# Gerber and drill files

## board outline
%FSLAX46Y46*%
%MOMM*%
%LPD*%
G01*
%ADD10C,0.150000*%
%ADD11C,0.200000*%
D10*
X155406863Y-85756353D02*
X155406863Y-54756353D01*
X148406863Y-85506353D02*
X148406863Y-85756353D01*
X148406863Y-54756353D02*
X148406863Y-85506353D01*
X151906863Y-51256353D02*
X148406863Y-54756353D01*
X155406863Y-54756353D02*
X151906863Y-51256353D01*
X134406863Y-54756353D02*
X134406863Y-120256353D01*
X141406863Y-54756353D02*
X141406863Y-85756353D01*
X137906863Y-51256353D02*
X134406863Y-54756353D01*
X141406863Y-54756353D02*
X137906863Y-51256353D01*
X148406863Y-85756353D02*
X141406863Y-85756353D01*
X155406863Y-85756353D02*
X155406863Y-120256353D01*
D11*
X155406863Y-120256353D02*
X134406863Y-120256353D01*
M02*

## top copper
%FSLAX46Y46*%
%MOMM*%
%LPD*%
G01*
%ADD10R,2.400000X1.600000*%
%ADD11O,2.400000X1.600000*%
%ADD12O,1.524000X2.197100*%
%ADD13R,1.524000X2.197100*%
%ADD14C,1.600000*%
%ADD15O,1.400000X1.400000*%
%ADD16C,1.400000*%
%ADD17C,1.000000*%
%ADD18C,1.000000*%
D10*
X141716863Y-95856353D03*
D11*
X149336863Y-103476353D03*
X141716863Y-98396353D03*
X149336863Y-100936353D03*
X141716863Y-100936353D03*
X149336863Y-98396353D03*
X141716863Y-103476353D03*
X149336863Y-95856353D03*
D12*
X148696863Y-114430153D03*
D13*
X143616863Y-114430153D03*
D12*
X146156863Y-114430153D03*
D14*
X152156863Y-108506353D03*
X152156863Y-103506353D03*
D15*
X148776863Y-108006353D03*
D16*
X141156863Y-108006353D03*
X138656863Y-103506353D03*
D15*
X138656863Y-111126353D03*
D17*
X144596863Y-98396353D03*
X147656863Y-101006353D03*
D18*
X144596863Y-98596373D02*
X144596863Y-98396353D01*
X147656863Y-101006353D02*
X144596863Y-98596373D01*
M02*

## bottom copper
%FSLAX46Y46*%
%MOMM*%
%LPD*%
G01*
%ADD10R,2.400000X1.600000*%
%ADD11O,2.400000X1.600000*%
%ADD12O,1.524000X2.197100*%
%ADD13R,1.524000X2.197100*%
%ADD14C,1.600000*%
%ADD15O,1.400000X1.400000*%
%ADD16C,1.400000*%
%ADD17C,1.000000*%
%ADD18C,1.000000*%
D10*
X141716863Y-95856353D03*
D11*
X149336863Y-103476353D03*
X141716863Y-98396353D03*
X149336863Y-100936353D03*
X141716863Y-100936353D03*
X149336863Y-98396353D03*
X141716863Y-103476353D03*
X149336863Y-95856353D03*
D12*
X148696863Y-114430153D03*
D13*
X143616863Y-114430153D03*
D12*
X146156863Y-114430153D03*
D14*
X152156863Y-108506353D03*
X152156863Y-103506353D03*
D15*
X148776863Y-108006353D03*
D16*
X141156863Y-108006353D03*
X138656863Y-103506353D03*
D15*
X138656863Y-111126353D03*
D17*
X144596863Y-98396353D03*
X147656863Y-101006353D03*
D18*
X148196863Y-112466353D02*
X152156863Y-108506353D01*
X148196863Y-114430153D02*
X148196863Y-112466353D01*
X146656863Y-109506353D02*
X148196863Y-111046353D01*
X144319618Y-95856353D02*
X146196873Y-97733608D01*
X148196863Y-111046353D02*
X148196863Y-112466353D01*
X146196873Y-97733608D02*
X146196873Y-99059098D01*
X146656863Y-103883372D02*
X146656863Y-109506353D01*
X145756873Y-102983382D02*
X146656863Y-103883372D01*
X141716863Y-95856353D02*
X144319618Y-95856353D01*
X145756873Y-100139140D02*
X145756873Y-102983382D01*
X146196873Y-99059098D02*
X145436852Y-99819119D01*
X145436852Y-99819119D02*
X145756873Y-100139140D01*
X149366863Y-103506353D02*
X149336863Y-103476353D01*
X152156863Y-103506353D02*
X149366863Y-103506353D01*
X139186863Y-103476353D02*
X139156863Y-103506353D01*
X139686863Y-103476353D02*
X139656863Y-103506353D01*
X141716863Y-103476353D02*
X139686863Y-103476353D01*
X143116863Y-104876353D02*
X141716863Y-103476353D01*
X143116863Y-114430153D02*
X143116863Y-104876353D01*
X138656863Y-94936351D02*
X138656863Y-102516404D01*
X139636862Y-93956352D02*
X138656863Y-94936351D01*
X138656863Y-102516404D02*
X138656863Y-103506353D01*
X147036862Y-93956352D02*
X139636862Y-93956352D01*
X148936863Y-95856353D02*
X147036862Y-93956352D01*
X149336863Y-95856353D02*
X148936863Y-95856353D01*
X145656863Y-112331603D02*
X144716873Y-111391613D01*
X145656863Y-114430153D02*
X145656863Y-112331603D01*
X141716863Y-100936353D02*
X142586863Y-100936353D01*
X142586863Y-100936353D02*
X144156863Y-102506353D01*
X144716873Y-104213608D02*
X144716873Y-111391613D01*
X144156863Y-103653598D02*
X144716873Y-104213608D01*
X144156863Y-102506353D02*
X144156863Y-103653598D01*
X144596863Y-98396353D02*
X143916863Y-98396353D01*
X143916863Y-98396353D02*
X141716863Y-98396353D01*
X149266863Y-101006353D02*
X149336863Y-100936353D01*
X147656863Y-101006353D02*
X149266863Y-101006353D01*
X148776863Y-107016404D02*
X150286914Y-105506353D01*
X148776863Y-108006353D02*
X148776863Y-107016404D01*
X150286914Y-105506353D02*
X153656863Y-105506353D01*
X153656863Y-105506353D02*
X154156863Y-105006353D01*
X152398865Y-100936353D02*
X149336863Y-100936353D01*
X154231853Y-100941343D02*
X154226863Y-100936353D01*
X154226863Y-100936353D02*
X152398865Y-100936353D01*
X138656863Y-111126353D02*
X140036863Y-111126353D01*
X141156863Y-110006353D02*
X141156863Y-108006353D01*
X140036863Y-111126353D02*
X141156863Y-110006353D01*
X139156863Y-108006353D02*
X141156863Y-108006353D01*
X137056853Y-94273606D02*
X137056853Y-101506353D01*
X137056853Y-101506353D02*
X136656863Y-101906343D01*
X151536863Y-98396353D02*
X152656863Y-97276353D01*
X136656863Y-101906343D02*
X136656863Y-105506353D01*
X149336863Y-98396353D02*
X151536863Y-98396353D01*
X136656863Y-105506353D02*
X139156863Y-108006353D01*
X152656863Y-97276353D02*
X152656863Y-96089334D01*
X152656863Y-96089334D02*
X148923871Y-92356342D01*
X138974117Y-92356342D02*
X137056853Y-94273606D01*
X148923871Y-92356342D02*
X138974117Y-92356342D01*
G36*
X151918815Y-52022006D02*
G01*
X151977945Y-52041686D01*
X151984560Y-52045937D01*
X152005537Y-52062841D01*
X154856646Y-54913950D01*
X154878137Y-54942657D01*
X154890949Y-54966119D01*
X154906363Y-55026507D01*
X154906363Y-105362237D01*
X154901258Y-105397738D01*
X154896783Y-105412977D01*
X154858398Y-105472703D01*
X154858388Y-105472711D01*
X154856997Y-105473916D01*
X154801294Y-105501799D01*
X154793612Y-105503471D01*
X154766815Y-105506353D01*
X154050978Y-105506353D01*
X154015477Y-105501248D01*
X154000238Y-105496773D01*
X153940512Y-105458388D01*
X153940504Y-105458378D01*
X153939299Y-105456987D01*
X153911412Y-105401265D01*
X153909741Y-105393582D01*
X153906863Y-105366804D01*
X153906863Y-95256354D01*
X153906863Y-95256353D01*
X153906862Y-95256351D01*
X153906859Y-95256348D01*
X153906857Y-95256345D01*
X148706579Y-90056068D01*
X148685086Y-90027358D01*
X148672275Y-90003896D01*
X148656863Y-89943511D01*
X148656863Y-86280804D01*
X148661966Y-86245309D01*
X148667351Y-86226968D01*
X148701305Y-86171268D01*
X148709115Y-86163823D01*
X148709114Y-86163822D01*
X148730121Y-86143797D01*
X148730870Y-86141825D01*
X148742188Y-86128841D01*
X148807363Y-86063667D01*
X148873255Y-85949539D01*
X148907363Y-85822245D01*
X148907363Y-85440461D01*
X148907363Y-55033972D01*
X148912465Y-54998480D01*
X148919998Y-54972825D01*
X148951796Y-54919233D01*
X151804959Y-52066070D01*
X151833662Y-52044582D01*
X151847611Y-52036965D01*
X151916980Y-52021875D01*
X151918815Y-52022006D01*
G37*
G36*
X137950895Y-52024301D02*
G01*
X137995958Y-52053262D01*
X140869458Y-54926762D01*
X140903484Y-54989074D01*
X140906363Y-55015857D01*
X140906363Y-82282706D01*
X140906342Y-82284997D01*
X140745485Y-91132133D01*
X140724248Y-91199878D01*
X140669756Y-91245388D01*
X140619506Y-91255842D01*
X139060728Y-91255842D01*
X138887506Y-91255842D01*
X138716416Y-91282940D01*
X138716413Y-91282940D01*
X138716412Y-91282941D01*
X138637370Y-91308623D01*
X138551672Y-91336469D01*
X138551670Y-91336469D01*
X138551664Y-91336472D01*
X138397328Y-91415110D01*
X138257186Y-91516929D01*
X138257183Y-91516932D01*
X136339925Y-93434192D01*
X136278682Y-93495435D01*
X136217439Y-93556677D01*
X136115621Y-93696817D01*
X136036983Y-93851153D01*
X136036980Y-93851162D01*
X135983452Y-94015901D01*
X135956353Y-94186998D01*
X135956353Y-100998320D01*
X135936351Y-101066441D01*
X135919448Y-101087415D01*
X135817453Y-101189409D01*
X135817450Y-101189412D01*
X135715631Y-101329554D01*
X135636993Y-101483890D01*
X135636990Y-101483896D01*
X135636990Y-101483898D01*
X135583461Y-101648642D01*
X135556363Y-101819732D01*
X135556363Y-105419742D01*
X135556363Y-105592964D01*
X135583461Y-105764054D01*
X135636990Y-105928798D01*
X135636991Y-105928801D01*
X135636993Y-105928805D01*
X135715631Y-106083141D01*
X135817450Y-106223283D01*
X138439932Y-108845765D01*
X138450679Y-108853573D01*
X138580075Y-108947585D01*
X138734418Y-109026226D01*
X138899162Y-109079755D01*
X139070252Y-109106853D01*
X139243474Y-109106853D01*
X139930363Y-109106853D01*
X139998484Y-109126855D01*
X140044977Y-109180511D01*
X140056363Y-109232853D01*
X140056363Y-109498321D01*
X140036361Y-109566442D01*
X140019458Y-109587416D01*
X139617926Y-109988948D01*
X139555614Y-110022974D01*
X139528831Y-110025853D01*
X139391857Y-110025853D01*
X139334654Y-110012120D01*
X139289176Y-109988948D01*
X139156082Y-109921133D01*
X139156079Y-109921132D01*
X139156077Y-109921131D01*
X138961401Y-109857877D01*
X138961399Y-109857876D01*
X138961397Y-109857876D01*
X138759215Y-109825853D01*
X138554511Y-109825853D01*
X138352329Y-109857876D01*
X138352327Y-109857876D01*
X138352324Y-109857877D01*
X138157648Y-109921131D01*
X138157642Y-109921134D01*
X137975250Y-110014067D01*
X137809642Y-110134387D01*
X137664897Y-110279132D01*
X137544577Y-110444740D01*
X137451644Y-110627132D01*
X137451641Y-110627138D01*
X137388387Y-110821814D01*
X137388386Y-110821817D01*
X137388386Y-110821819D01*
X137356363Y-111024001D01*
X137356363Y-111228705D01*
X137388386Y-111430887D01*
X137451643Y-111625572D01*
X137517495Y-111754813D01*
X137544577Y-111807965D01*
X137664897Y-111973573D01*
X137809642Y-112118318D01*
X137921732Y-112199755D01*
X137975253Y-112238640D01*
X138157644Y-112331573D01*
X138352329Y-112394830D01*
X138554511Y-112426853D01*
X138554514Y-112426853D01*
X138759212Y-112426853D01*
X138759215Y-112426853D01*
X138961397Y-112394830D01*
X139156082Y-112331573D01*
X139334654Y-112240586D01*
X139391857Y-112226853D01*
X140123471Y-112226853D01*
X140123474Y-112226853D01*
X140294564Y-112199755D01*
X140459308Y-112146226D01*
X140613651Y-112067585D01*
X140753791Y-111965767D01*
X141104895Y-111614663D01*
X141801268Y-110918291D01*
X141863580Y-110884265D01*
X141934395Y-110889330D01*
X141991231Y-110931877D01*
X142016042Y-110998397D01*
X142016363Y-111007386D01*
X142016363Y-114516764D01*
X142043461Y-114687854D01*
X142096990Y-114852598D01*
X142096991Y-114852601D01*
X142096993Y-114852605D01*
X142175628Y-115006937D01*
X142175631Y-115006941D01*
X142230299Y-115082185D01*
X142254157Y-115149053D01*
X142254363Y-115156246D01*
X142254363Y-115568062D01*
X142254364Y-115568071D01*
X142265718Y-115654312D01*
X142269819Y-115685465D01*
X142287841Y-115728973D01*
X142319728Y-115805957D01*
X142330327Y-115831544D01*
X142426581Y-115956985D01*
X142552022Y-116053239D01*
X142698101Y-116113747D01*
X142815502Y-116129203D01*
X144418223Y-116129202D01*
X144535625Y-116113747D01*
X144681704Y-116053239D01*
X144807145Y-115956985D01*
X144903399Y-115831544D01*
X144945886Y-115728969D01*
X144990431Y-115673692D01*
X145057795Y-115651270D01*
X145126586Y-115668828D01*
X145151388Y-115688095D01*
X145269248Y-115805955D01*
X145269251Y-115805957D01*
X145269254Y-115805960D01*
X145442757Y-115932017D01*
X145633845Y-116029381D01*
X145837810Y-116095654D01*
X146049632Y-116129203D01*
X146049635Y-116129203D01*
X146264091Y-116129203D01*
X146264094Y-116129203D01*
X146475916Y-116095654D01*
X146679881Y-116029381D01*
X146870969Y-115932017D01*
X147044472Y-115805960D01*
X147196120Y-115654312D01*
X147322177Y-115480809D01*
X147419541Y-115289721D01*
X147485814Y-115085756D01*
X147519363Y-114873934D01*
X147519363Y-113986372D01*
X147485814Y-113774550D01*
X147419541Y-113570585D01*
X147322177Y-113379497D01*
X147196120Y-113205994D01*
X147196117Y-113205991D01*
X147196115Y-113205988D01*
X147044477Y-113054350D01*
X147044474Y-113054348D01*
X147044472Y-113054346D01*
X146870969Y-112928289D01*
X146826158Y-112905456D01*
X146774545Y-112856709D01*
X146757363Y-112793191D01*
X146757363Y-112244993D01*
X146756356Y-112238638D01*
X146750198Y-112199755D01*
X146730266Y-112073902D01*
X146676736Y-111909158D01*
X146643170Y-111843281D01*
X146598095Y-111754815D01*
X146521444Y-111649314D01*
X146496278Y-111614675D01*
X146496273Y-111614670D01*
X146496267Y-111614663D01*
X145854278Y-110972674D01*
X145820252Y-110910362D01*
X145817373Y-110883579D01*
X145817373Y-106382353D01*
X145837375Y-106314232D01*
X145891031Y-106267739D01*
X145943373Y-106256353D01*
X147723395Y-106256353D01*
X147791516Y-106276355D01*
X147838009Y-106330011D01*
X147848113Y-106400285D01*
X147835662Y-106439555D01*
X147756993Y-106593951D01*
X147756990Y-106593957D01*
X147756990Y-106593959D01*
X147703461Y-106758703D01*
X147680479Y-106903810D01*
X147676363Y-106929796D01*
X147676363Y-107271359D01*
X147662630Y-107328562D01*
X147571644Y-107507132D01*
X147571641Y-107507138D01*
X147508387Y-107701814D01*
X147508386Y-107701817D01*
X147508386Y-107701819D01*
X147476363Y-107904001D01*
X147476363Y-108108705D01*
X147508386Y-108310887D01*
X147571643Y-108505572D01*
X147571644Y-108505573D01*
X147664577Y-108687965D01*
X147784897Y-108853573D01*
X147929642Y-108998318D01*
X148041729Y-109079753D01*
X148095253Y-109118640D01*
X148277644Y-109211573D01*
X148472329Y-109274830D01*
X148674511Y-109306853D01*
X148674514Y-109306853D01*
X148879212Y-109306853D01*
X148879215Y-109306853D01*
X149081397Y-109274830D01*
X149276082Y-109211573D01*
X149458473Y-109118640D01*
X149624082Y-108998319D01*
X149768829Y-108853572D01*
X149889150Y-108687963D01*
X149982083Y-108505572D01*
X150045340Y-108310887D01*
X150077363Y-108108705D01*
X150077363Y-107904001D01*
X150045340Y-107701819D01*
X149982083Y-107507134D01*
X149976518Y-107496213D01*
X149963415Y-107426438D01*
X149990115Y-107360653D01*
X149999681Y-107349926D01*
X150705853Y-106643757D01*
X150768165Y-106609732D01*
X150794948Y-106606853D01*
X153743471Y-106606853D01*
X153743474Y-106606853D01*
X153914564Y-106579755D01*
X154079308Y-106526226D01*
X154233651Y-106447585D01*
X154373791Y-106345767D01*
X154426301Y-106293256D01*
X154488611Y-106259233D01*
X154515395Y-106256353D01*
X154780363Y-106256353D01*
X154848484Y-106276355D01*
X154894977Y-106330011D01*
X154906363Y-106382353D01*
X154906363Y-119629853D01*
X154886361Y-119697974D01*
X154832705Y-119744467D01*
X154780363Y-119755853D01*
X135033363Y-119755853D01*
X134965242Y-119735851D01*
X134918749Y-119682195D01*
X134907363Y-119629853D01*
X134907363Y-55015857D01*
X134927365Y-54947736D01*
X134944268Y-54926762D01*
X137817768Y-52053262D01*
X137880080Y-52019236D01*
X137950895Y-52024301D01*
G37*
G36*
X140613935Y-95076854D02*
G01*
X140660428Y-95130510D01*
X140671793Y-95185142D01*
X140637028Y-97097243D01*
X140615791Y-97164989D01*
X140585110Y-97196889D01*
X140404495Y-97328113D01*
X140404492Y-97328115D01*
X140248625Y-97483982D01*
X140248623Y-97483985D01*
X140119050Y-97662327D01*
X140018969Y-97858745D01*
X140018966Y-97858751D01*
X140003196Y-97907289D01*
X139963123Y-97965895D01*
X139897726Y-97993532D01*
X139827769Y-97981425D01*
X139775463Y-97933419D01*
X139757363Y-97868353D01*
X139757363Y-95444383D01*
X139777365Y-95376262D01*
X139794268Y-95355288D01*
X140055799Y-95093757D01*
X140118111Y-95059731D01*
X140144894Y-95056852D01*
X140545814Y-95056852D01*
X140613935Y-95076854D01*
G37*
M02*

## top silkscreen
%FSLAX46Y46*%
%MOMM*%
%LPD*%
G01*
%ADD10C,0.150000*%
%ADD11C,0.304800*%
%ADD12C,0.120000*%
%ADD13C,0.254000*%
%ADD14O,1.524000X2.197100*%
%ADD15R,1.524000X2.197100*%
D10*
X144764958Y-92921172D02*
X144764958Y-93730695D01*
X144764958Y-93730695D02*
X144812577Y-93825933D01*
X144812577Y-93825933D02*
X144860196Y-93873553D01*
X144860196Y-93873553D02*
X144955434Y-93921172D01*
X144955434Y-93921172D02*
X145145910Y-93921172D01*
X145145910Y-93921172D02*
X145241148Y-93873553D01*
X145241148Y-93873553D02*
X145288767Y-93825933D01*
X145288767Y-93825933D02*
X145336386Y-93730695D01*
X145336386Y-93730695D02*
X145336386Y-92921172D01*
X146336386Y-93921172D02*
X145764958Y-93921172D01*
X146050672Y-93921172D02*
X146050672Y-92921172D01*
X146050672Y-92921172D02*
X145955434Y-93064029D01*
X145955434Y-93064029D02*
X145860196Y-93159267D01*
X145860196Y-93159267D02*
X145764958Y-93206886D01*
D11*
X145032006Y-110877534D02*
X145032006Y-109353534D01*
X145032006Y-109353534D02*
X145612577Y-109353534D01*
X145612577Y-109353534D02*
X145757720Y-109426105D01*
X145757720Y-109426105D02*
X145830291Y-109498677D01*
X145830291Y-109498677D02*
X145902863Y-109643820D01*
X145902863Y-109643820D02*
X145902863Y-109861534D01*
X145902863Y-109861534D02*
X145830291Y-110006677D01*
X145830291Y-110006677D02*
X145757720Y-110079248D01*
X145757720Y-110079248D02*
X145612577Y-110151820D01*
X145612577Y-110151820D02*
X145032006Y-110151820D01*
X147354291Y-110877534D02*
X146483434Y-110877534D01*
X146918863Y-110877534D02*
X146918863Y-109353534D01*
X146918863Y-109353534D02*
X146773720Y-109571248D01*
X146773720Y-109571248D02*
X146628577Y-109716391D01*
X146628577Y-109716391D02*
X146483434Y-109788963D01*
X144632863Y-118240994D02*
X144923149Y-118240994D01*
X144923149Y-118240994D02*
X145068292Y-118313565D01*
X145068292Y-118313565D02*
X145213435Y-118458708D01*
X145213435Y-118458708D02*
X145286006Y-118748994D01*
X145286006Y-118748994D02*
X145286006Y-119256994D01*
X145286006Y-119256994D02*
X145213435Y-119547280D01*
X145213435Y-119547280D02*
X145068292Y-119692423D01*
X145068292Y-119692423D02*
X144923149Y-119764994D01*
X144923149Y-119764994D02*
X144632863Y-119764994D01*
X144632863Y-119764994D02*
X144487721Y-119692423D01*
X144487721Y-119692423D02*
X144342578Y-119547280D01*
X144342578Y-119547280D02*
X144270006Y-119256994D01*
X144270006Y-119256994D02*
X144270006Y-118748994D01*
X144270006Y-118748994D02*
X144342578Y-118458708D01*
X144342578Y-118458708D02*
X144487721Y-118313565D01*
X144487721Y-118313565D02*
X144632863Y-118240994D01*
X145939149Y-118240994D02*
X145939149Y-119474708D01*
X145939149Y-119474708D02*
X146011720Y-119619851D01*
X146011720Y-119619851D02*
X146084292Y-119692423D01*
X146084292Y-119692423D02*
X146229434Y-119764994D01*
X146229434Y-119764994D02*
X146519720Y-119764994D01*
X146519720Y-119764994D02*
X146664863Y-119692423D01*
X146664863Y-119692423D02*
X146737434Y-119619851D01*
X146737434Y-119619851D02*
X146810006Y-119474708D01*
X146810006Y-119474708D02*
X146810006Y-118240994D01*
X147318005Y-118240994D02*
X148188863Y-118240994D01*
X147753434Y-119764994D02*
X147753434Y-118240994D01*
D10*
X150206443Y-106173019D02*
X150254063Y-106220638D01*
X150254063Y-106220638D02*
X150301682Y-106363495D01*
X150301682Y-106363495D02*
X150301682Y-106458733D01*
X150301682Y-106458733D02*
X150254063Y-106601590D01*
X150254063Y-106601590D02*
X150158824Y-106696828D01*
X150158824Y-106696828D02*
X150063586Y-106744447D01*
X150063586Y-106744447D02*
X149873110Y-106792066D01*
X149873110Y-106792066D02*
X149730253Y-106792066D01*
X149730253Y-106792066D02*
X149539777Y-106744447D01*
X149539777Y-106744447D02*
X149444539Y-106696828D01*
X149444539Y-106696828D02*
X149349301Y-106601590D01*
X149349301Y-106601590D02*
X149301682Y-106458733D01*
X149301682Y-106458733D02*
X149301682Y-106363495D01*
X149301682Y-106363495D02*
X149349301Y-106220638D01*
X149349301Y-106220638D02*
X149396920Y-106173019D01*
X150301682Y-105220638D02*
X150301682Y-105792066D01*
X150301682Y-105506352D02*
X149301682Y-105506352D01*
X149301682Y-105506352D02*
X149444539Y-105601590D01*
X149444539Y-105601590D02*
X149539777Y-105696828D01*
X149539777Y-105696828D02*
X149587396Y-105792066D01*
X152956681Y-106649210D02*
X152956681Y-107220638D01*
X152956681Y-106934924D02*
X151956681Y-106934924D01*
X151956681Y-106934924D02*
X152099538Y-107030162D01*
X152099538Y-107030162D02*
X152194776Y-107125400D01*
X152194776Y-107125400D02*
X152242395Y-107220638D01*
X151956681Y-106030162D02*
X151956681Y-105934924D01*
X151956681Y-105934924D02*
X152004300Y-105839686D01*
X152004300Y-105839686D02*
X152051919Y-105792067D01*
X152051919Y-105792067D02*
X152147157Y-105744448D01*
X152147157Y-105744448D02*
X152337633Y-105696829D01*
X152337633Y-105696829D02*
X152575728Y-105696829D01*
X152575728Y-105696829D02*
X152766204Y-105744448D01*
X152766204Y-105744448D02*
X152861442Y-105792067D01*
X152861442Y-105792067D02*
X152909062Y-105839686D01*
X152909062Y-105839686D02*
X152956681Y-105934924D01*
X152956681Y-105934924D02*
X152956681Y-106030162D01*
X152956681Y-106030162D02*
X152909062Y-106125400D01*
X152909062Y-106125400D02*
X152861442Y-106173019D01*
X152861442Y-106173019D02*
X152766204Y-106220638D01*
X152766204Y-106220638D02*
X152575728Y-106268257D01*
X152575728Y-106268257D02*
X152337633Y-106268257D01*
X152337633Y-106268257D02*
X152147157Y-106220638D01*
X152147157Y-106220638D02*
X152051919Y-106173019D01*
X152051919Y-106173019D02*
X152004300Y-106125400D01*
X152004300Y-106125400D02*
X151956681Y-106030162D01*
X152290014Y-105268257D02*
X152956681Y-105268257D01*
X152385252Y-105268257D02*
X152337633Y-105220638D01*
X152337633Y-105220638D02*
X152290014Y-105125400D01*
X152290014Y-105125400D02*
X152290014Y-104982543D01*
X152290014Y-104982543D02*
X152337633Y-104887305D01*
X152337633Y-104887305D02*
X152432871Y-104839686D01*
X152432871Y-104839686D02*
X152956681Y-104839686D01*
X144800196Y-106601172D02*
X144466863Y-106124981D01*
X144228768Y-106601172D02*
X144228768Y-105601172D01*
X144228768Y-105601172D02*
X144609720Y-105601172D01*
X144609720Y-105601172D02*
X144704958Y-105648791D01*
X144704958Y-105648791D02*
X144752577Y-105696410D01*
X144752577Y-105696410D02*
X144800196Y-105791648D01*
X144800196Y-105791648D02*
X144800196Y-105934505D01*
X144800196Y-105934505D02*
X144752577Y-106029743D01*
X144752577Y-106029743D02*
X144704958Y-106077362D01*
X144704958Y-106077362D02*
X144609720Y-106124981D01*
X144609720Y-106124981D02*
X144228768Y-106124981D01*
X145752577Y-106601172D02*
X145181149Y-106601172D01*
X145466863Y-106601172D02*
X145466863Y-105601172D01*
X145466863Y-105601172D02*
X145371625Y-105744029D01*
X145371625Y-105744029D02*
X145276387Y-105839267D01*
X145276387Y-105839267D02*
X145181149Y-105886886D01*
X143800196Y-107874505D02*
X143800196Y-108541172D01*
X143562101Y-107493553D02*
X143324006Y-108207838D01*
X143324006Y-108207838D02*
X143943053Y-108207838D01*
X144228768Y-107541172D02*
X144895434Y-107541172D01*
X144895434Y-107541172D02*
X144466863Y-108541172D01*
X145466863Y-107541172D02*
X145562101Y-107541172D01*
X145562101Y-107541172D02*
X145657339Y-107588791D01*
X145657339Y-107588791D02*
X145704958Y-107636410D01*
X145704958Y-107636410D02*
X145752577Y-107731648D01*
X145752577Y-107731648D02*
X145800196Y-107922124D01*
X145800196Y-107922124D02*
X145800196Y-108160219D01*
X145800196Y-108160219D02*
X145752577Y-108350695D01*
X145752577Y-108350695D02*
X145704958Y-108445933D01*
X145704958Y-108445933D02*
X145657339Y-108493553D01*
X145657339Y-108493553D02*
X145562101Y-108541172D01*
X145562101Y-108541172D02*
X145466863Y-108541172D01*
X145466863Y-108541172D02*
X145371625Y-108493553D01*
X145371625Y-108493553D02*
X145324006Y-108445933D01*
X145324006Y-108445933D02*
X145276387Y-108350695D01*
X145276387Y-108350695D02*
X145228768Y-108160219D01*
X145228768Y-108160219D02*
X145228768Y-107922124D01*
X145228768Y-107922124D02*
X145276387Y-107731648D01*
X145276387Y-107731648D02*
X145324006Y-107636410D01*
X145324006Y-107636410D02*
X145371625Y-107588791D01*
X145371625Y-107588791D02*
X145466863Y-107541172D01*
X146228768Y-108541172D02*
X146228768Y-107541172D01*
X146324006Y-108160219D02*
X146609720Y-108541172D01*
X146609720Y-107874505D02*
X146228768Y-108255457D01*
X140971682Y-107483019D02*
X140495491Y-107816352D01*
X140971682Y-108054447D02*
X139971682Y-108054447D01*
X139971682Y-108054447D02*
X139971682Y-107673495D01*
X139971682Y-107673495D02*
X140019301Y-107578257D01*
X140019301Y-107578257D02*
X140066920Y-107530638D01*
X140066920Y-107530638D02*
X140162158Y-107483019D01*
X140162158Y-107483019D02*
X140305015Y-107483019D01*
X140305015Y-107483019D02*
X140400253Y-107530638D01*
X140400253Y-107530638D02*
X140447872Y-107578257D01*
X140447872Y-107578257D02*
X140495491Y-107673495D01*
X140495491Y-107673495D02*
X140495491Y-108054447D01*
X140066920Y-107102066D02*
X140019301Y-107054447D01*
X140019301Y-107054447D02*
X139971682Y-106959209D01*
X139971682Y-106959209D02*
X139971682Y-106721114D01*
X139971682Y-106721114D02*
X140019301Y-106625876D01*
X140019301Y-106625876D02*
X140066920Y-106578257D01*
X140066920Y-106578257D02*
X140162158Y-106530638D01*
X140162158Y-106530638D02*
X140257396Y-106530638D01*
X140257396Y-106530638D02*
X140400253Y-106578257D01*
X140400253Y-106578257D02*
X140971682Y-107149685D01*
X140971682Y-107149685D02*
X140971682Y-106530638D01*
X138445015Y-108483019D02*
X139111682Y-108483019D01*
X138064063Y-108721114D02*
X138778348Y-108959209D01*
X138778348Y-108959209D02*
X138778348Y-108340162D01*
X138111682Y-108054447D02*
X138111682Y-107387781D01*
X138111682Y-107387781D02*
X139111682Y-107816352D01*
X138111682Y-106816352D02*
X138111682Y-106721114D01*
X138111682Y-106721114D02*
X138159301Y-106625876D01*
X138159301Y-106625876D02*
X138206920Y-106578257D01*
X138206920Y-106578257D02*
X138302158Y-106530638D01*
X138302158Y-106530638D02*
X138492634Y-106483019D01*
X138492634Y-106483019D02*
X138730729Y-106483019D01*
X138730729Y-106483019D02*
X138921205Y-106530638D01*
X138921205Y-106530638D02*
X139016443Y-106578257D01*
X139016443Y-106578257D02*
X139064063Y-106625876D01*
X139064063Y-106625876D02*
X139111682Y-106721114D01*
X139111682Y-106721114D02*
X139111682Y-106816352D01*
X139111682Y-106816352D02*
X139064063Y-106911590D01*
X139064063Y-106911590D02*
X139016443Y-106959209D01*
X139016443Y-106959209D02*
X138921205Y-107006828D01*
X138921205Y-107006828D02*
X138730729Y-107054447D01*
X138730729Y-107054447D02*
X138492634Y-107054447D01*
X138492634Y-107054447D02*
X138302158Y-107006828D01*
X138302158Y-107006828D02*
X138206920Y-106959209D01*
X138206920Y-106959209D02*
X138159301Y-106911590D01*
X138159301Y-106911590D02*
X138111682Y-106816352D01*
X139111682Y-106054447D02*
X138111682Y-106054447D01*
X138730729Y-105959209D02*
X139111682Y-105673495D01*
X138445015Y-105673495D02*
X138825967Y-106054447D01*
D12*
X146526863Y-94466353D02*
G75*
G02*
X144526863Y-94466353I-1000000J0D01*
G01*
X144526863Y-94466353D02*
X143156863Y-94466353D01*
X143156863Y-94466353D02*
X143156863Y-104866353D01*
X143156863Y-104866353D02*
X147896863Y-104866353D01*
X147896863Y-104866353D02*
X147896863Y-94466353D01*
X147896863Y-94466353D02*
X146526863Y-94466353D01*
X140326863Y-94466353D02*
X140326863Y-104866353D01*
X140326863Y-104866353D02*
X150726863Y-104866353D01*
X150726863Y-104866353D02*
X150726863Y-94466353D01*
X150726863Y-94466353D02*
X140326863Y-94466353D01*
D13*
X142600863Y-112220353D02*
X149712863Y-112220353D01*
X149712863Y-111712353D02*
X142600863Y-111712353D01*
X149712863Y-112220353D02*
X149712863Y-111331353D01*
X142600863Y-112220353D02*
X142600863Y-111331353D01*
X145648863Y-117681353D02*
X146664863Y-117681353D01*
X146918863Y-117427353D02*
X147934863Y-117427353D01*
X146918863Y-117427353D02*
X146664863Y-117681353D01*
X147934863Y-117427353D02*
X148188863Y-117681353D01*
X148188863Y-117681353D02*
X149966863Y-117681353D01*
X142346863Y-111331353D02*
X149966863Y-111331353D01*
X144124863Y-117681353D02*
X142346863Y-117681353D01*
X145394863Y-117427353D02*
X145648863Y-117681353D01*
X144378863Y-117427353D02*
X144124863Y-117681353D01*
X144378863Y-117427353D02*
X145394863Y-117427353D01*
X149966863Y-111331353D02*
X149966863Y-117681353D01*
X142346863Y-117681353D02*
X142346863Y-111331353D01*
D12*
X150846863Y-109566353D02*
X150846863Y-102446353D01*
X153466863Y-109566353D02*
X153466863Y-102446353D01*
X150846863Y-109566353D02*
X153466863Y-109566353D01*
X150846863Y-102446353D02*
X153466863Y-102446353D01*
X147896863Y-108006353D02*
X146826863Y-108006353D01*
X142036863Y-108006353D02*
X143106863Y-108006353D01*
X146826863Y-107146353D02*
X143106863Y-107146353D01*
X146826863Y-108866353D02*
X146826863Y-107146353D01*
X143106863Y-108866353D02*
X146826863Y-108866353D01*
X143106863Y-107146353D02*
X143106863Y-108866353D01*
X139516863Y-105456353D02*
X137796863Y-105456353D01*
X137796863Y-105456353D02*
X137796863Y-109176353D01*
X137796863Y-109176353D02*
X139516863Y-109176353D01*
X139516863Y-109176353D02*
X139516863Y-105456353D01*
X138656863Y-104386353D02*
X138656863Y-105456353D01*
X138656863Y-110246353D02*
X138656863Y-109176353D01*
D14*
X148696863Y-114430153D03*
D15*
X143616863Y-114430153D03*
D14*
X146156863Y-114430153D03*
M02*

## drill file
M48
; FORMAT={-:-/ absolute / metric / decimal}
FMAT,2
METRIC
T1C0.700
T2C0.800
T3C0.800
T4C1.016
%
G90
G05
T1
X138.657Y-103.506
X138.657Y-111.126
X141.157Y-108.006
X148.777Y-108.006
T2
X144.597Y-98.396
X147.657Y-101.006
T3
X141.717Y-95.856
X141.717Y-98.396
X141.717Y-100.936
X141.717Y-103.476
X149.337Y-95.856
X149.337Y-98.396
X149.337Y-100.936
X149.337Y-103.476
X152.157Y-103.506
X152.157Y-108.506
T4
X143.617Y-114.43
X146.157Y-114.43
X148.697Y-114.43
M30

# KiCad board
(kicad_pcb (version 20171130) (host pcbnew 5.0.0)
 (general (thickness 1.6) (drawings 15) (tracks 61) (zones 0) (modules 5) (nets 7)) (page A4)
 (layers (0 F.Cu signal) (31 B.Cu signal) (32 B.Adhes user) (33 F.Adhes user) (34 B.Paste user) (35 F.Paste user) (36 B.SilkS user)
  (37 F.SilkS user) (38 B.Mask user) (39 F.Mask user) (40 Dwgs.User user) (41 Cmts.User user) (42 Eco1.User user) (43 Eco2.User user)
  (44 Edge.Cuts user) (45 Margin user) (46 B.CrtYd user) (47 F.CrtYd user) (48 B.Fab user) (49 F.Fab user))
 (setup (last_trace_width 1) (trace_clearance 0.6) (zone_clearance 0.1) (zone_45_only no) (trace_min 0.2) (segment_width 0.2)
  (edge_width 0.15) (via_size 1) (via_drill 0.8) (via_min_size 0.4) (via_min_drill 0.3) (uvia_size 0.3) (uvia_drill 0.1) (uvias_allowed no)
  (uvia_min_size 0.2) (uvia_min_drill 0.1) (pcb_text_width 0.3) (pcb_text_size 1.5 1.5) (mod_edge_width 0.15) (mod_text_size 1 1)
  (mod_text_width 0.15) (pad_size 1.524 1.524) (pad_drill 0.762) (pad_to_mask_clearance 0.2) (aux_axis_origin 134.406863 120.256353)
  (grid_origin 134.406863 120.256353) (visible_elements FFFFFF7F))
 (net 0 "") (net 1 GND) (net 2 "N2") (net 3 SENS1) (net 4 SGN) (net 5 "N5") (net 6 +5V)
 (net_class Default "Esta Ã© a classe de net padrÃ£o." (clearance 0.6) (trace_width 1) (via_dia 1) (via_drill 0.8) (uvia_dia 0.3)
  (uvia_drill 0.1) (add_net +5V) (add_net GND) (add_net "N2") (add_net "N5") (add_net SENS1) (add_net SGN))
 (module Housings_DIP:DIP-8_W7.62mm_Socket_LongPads (layer F.Cu) (at 141.716863 95.856353)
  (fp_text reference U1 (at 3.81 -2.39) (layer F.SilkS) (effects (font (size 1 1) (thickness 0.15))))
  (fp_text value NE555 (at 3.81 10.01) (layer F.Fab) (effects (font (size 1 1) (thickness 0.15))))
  (fp_arc (start 3.81 -1.39) (end 2.81 -1.39) (angle -180) (layer F.SilkS) (width 0.12))
  (fp_line (start 2.81 -1.39) (end 1.44 -1.39) (layer F.SilkS) (width 0.12))
  (fp_line (start 1.44 -1.39) (end 1.44 9.01) (layer F.SilkS) (width 0.12))
  (fp_line (start 1.44 9.01) (end 6.18 9.01) (layer F.SilkS) (width 0.12))
  (fp_line (start 6.18 9.01) (end 6.18 -1.39) (layer F.SilkS) (width 0.12))
  (fp_line (start 6.18 -1.39) (end 4.81 -1.39) (layer F.SilkS) (width 0.12))
  (fp_line (start -1.39 -1.39) (end -1.39 9.01) (layer F.SilkS) (width 0.12))
  (fp_line (start -1.39 9.01) (end 9.01 9.01) (layer F.SilkS) (width 0.12))
  (fp_line (start 9.01 9.01) (end 9.01 -1.39) (layer F.SilkS) (width 0.12))
  (fp_line (start 9.01 -1.39) (end -1.39 -1.39) (layer F.SilkS) (width 0.12))
  (pad 1 thru_hole rect (at 0 0) (size 2.4 1.6) (drill 0.8) (layers *.Mask B.Cu) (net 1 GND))
  (pad 5 thru_hole oval (at 7.62 7.62) (size 2.4 1.6) (drill 0.8) (layers *.Mask B.Cu) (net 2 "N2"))
  (pad 2 thru_hole oval (at 0 2.54) (size 2.4 1.6) (drill 0.8) (layers *.Mask B.Cu) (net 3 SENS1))
  (pad 6 thru_hole oval (at 7.62 5.08) (size 2.4 1.6) (drill 0.8) (layers *.Mask B.Cu) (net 3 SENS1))
  (pad 3 thru_hole oval (at 0 5.08) (size 2.4 1.6) (drill 0.8) (layers *.Mask B.Cu) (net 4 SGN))
  (pad 7 thru_hole oval (at 7.62 2.54) (size 2.4 1.6) (drill 0.8) (layers *.Mask B.Cu) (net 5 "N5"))
  (pad 4 thru_hole oval (at 0 7.62) (size 2.4 1.6) (drill 0.8) (layers *.Mask B.Cu) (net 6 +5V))
  (pad 8 thru_hole oval (at 7.62 0) (size 2.4 1.6) (drill 0.8) (layers *.Mask B.Cu) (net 6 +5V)))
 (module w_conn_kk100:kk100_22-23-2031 (layer F.Cu) (at 146.156863 114.506353)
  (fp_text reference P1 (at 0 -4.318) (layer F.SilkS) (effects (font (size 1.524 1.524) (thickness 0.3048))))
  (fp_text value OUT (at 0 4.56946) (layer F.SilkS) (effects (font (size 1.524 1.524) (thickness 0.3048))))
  (fp_line (start -3.556 -2.286) (end 3.556 -2.286) (layer F.SilkS) (width 0.254))
  (fp_line (start 3.556 -2.794) (end -3.556 -2.794) (layer F.SilkS) (width 0.254))
  (fp_line (start 3.556 -2.286) (end 3.556 -3.175) (layer F.SilkS) (width 0.254))
  (fp_line (start -3.556 -2.286) (end -3.556 -3.175) (layer F.SilkS) (width 0.254))
  (fp_line (start -0.508 3.175) (end 0.508 3.175) (layer F.SilkS) (width 0.254))
  (fp_line (start 0.762 2.921) (end 1.778 2.921) (layer F.SilkS) (width 0.254))
  (fp_line (start 0.762 2.921) (end 0.508 3.175) (layer F.SilkS) (width 0.254))
  (fp_line (start 1.778 2.921) (end 2.032 3.175) (layer F.SilkS) (width 0.254))
  (fp_line (start 2.032 3.175) (end 3.81 3.175) (layer F.SilkS) (width 0.254))
  (fp_line (start -3.81 -3.175) (end 3.81 -3.175) (layer F.SilkS) (width 0.254))
  (fp_line (start -2.032 3.175) (end -3.81 3.175) (layer F.SilkS) (width 0.254))
  (fp_line (start -0.762 2.921) (end -0.508 3.175) (layer F.SilkS) (width 0.254))
  (fp_line (start -1.778 2.921) (end -2.032 3.175) (layer F.SilkS) (width 0.254))
  (fp_line (start -1.778 2.921) (end -0.762 2.921) (layer F.SilkS) (width 0.254))
  (fp_line (start 3.81 -3.175) (end 3.81 3.175) (layer F.SilkS) (width 0.254))
  (fp_line (start -3.81 3.175) (end -3.81 -3.175) (layer F.SilkS) (width 0.254))
  (pad 3 thru_hole oval (at 2.54 -0.0762) (size 1.524 2.1971) (drill 1.016) (layers *.Cu *.Mask F.SilkS) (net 1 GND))
  (pad 1 thru_hole rect (at -2.54 -0.0762) (size 1.524 2.1971) (drill 1.016) (layers *.Cu *.Mask F.SilkS) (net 6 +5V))
  (pad 2 thru_hole oval (at 0 -0.0762) (size 1.524 2.1971) (drill 1.016) (layers *.Cu *.Mask F.SilkS) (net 4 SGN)))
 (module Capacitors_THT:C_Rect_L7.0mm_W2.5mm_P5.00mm (layer F.Cu) (at 152.156863 108.506353 90)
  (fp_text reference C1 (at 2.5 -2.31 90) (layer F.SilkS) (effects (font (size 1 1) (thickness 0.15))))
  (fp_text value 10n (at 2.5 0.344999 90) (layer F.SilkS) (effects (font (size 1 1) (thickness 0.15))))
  (fp_line (start -1.06 -1.31) (end 6.06 -1.31) (layer F.SilkS) (width 0.12))
  (fp_line (start -1.06 1.31) (end 6.06 1.31) (layer F.SilkS) (width 0.12))
  (fp_line (start -1.06 -1.31) (end -1.06 1.31) (layer F.SilkS) (width 0.12))
  (fp_line (start 6.06 -1.31) (end 6.06 1.31) (layer F.SilkS) (width 0.12))
  (pad 1 thru_hole circle (at 0 0 90) (size 1.6 1.6) (drill 0.8) (layers *.Mask B.Cu) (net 1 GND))
  (pad 2 thru_hole circle (at 5 0 90) (size 1.6 1.6) (drill 0.8) (layers *.Mask B.Cu) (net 2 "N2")))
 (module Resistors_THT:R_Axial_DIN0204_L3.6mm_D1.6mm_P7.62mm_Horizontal (layer F.Cu) (at 141.156863 108.006353)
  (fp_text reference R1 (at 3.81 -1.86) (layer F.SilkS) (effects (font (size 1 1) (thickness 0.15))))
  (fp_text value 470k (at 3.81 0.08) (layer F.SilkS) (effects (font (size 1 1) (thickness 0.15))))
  (fp_line (start 6.74 0) (end 5.67 0) (layer F.SilkS) (width 0.12))
  (fp_line (start 0.88 0) (end 1.95 0) (layer F.SilkS) (width 0.12))
  (fp_line (start 5.67 -0.86) (end 1.95 -0.86) (layer F.SilkS) (width 0.12))
  (fp_line (start 5.67 0.86) (end 5.67 -0.86) (layer F.SilkS) (width 0.12))
  (fp_line (start 1.95 0.86) (end 5.67 0.86) (layer F.SilkS) (width 0.12))
  (fp_line (start 1.95 -0.86) (end 1.95 0.86) (layer F.SilkS) (width 0.12))
  (pad 2 thru_hole oval (at 7.62 0) (size 1.4 1.4) (drill 0.7) (layers *.Cu *.Mask) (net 3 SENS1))
  (pad 1 thru_hole circle (at 0 0) (size 1.4 1.4) (drill 0.7) (layers *.Cu *.Mask) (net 5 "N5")))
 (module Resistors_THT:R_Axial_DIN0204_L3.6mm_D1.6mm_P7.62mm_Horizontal (layer F.Cu) (at 138.656863 103.506353 270)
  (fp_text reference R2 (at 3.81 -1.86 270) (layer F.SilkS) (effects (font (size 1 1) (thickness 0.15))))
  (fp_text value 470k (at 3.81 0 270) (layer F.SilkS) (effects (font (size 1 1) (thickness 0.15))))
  (fp_line (start 1.95 -0.86) (end 1.95 0.86) (layer F.SilkS) (width 0.12))
  (fp_line (start 1.95 0.86) (end 5.67 0.86) (layer F.SilkS) (width 0.12))
  (fp_line (start 5.67 0.86) (end 5.67 -0.86) (layer F.SilkS) (width 0.12))
  (fp_line (start 5.67 -0.86) (end 1.95 -0.86) (layer F.SilkS) (width 0.12))
  (fp_line (start 0.88 0) (end 1.95 0) (layer F.SilkS) (width 0.12))
  (fp_line (start 6.74 0) (end 5.67 0) (layer F.SilkS) (width 0.12))
  (pad 1 thru_hole circle (at 0 0 270) (size 1.4 1.4) (drill 0.7) (layers *.Cu *.Mask) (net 6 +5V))
  (pad 2 thru_hole oval (at 7.62 0 270) (size 1.4 1.4) (drill 0.7) (layers *.Cu *.Mask) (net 5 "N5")))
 (gr_line (start 155.406863 85.756353) (end 155.406863 54.756353) (layer Edge.Cuts) (width 0.15))
 (gr_line (start 148.406863 85.506353) (end 148.406863 85.756353) (layer Edge.Cuts) (width 0.15))
 (gr_line (start 148.406863 54.756353) (end 148.406863 85.506353) (layer Edge.Cuts) (width 0.15))
 (gr_line (start 151.906863 51.256353) (end 148.406863 54.756353) (layer Edge.Cuts) (width 0.15))
 (gr_line (start 155.406863 54.756353) (end 151.906863 51.256353) (layer Edge.Cuts) (width 0.15))
 (gr_line (start 134.406863 54.756353) (end 134.406863 120.256353) (layer Edge.Cuts) (width 0.15))
 (gr_line (start 141.406863 54.756353) (end 141.406863 85.756353) (layer Edge.Cuts) (width 0.15))
 (gr_line (start 137.906863 51.256353) (end 134.406863 54.756353) (layer Edge.Cuts) (width 0.15))
 (gr_line (start 141.406863 54.756353) (end 137.906863 51.256353) (layer Edge.Cuts) (width 0.15))
 (gr_line (start 148.406863 85.756353) (end 141.406863 85.756353) (layer Edge.Cuts) (width 0.15))
 (gr_line (start 155.406863 85.756353) (end 155.406863 120.256353) (layer Edge.Cuts) (width 0.15))
 (gr_line (start 155.406863 120.256353) (end 134.406863 120.256353) (layer Edge.Cuts) (width 0.2))
 (segment (start 148.196863 112.466353) (end 152.156863 108.506353) (width 1) (layer B.Cu) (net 1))
 (segment (start 148.196863 114.430153) (end 148.196863 112.466353) (width 1) (layer B.Cu) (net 1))
 (segment (start 146.656863 109.506353) (end 148.196863 111.046353) (width 1) (layer B.Cu) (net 1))
 (segment (start 144.319618 95.856353) (end 146.196873 97.733608) (width 1) (layer B.Cu) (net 1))
 (segment (start 148.196863 111.046353) (end 148.196863 112.466353) (width 1) (layer B.Cu) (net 1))
 (segment (start 146.196873 97.733608) (end 146.196873 99.059098) (width 1) (layer B.Cu) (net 1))
 (segment (start 146.656863 103.883372) (end 146.656863 109.506353) (width 1) (layer B.Cu) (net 1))
 (segment (start 145.756873 102.983382) (end 146.656863 103.883372) (width 1) (layer B.Cu) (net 1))
 (segment (start 141.716863 95.856353) (end 144.319618 95.856353) (width 1) (layer B.Cu) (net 1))
 (segment (start 145.756873 100.13914) (end 145.756873 102.983382) (width 1) (layer B.Cu) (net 1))
 (segment (start 146.196873 99.059098) (end 145.436852 99.819119) (width 1) (layer B.Cu) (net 1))
 (segment (start 145.436852 99.819119) (end 145.756873 100.13914) (width 1) (layer B.Cu) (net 1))
 (segment (start 149.366863 103.506353) (end 149.336863 103.476353) (width 1) (layer B.Cu) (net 2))
 (segment (start 152.156863 103.506353) (end 149.366863 103.506353) (width 1) (layer B.Cu) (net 2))
 (segment (start 139.186863 103.476353) (end 139.156863 103.506353) (width 1) (layer B.Cu) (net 6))
 (segment (start 139.686863 103.476353) (end 139.656863 103.506353) (width 1) (layer B.Cu) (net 6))
 (segment (start 141.716863 103.476353) (end 139.686863 103.476353) (width 1) (layer B.Cu) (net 6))
 (segment (start 143.116863 104.876353) (end 141.716863 103.476353) (width 1) (layer B.Cu) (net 6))
 (segment (start 143.116863 114.430153) (end 143.116863 104.876353) (width 1) (layer B.Cu) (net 6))
 (segment (start 138.656863 94.936351) (end 138.656863 102.516404) (width 1) (layer B.Cu) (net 6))
 (segment (start 139.636862 93.956352) (end 138.656863 94.936351) (width 1) (layer B.Cu) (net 6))
 (segment (start 138.656863 102.516404) (end 138.656863 103.506353) (width 1) (layer B.Cu) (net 6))
 (segment (start 147.036862 93.956352) (end 139.636862 93.956352) (width 1) (layer B.Cu) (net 6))
 (segment (start 148.936863 95.856353) (end 147.036862 93.956352) (width 1) (layer B.Cu) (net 6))
 (segment (start 149.336863 95.856353) (end 148.936863 95.856353) (width 1) (layer B.Cu) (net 6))
 (segment (start 145.656863 112.331603) (end 144.716873 111.391613) (width 1) (layer B.Cu) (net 4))
 (segment (start 145.656863 114.430153) (end 145.656863 112.331603) (width 1) (layer B.Cu) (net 4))
 (segment (start 141.716863 100.936353) (end 142.586863 100.936353) (width 1) (layer B.Cu) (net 4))
 (segment (start 142.586863 100.936353) (end 144.156863 102.506353) (width 1) (layer B.Cu) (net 4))
 (segment (start 144.716873 104.213608) (end 144.716873 111.391613) (width 1) (layer B.Cu) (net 4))
 (segment (start 144.156863 103.653598) (end 144.716873 104.213608) (width 1) (layer B.Cu) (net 4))
 (segment (start 144.156863 102.506353) (end 144.156863 103.653598) (width 1) (layer B.Cu) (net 4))
 (segment (start 144.596863 98.396353) (end 143.916863 98.396353) (width 1) (layer B.Cu) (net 3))
 (segment (start 143.916863 98.396353) (end 141.716863 98.396353) (width 1) (layer B.Cu) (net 3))
 (via (at 144.596863 98.396353) (size 1) (drill 0.8) (layers F.Cu B.Cu) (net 3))
 (segment (start 144.596863 98.596373) (end 144.596863 98.396353) (width 1) (layer F.Cu) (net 3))
 (via (at 147.656863 101.006353) (size 1) (drill 0.8) (layers F.Cu B.Cu) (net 3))
 (segment (start 147.656863 101.006353) (end 144.596863 98.596373) (width 1) (layer F.Cu) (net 3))
 (segment (start 149.266863 101.006353) (end 149.336863 100.936353) (width 1) (layer B.Cu) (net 3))
 (segment (start 147.656863 101.006353) (end 149.266863 101.006353) (width 1) (layer B.Cu) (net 3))
 (segment (start 148.776863 107.016404) (end 150.286914 105.506353) (width 1) (layer B.Cu) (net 3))
 (segment (start 148.776863 108.006353) (end 148.776863 107.016404) (width 1) (layer B.Cu) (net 3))
 (segment (start 150.286914 105.506353) (end 153.656863 105.506353) (width 1) (layer B.Cu) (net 3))
 (segment (start 153.656863 105.506353) (end 154.156863 105.006353) (width 1) (layer B.Cu) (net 3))
 (segment (start 152.398865 100.936353) (end 149.336863 100.936353) (width 1) (layer B.Cu) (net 3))
 (segment (start 154.231853 100.941343) (end 154.226863 100.936353) (width 1) (layer B.Cu) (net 3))
 (segment (start 154.226863 100.936353) (end 152.398865 100.936353) (width 1) (layer B.Cu) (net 3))
 (segment (start 138.656863 111.126353) (end 140.036863 111.126353) (width 1) (layer B.Cu) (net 5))
 (segment (start 141.156863 110.006353) (end 141.156863 108.006353) (width 1) (layer B.Cu) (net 5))
 (segment (start 140.036863 111.126353) (end 141.156863 110.006353) (width 1) (layer B.Cu) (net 5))
 (segment (start 139.156863 108.006353) (end 141.156863 108.006353) (width 1) (layer B.Cu) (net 5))
 (segment (start 137.056853 94.273606) (end 137.056853 101.506353) (width 1) (layer B.Cu) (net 5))
 (segment (start 137.056853 101.506353) (end 136.656863 101.906343) (width 1) (layer B.Cu) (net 5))
 (segment (start 151.536863 98.396353) (end 152.656863 97.276353) (width 1) (layer B.Cu) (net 5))
 (segment (start 136.656863 101.906343) (end 136.656863 105.506353) (width 1) (layer B.Cu) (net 5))
 (segment (start 149.336863 98.396353) (end 151.536863 98.396353) (width 1) (layer B.Cu) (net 5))
 (segment (start 136.656863 105.506353) (end 139.156863 108.006353) (width 1) (layer B.Cu) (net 5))
 (segment (start 152.656863 97.276353) (end 152.656863 96.089334) (width 1) (layer B.Cu) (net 5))
 (segment (start 152.656863 96.089334) (end 148.923871 92.356342) (width 1) (layer B.Cu) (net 5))
 (segment (start 138.974117 92.356342) (end 137.056853 94.273606) (width 1) (layer B.Cu) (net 5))
 (segment (start 148.923871 92.356342) (end 138.974117 92.356342) (width 1) (layer B.Cu) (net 5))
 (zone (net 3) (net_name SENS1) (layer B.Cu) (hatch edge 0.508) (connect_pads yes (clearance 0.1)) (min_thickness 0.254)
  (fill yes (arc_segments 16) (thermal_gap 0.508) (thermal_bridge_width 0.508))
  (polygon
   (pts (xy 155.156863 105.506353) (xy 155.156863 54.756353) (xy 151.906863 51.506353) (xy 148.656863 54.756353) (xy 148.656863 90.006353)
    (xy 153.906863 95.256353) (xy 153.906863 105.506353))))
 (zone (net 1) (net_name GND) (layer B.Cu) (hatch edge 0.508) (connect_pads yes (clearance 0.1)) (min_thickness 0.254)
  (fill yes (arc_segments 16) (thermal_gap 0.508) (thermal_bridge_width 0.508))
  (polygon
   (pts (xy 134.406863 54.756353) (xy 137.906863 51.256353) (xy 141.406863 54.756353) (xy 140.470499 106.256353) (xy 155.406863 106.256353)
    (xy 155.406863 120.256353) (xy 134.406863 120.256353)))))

